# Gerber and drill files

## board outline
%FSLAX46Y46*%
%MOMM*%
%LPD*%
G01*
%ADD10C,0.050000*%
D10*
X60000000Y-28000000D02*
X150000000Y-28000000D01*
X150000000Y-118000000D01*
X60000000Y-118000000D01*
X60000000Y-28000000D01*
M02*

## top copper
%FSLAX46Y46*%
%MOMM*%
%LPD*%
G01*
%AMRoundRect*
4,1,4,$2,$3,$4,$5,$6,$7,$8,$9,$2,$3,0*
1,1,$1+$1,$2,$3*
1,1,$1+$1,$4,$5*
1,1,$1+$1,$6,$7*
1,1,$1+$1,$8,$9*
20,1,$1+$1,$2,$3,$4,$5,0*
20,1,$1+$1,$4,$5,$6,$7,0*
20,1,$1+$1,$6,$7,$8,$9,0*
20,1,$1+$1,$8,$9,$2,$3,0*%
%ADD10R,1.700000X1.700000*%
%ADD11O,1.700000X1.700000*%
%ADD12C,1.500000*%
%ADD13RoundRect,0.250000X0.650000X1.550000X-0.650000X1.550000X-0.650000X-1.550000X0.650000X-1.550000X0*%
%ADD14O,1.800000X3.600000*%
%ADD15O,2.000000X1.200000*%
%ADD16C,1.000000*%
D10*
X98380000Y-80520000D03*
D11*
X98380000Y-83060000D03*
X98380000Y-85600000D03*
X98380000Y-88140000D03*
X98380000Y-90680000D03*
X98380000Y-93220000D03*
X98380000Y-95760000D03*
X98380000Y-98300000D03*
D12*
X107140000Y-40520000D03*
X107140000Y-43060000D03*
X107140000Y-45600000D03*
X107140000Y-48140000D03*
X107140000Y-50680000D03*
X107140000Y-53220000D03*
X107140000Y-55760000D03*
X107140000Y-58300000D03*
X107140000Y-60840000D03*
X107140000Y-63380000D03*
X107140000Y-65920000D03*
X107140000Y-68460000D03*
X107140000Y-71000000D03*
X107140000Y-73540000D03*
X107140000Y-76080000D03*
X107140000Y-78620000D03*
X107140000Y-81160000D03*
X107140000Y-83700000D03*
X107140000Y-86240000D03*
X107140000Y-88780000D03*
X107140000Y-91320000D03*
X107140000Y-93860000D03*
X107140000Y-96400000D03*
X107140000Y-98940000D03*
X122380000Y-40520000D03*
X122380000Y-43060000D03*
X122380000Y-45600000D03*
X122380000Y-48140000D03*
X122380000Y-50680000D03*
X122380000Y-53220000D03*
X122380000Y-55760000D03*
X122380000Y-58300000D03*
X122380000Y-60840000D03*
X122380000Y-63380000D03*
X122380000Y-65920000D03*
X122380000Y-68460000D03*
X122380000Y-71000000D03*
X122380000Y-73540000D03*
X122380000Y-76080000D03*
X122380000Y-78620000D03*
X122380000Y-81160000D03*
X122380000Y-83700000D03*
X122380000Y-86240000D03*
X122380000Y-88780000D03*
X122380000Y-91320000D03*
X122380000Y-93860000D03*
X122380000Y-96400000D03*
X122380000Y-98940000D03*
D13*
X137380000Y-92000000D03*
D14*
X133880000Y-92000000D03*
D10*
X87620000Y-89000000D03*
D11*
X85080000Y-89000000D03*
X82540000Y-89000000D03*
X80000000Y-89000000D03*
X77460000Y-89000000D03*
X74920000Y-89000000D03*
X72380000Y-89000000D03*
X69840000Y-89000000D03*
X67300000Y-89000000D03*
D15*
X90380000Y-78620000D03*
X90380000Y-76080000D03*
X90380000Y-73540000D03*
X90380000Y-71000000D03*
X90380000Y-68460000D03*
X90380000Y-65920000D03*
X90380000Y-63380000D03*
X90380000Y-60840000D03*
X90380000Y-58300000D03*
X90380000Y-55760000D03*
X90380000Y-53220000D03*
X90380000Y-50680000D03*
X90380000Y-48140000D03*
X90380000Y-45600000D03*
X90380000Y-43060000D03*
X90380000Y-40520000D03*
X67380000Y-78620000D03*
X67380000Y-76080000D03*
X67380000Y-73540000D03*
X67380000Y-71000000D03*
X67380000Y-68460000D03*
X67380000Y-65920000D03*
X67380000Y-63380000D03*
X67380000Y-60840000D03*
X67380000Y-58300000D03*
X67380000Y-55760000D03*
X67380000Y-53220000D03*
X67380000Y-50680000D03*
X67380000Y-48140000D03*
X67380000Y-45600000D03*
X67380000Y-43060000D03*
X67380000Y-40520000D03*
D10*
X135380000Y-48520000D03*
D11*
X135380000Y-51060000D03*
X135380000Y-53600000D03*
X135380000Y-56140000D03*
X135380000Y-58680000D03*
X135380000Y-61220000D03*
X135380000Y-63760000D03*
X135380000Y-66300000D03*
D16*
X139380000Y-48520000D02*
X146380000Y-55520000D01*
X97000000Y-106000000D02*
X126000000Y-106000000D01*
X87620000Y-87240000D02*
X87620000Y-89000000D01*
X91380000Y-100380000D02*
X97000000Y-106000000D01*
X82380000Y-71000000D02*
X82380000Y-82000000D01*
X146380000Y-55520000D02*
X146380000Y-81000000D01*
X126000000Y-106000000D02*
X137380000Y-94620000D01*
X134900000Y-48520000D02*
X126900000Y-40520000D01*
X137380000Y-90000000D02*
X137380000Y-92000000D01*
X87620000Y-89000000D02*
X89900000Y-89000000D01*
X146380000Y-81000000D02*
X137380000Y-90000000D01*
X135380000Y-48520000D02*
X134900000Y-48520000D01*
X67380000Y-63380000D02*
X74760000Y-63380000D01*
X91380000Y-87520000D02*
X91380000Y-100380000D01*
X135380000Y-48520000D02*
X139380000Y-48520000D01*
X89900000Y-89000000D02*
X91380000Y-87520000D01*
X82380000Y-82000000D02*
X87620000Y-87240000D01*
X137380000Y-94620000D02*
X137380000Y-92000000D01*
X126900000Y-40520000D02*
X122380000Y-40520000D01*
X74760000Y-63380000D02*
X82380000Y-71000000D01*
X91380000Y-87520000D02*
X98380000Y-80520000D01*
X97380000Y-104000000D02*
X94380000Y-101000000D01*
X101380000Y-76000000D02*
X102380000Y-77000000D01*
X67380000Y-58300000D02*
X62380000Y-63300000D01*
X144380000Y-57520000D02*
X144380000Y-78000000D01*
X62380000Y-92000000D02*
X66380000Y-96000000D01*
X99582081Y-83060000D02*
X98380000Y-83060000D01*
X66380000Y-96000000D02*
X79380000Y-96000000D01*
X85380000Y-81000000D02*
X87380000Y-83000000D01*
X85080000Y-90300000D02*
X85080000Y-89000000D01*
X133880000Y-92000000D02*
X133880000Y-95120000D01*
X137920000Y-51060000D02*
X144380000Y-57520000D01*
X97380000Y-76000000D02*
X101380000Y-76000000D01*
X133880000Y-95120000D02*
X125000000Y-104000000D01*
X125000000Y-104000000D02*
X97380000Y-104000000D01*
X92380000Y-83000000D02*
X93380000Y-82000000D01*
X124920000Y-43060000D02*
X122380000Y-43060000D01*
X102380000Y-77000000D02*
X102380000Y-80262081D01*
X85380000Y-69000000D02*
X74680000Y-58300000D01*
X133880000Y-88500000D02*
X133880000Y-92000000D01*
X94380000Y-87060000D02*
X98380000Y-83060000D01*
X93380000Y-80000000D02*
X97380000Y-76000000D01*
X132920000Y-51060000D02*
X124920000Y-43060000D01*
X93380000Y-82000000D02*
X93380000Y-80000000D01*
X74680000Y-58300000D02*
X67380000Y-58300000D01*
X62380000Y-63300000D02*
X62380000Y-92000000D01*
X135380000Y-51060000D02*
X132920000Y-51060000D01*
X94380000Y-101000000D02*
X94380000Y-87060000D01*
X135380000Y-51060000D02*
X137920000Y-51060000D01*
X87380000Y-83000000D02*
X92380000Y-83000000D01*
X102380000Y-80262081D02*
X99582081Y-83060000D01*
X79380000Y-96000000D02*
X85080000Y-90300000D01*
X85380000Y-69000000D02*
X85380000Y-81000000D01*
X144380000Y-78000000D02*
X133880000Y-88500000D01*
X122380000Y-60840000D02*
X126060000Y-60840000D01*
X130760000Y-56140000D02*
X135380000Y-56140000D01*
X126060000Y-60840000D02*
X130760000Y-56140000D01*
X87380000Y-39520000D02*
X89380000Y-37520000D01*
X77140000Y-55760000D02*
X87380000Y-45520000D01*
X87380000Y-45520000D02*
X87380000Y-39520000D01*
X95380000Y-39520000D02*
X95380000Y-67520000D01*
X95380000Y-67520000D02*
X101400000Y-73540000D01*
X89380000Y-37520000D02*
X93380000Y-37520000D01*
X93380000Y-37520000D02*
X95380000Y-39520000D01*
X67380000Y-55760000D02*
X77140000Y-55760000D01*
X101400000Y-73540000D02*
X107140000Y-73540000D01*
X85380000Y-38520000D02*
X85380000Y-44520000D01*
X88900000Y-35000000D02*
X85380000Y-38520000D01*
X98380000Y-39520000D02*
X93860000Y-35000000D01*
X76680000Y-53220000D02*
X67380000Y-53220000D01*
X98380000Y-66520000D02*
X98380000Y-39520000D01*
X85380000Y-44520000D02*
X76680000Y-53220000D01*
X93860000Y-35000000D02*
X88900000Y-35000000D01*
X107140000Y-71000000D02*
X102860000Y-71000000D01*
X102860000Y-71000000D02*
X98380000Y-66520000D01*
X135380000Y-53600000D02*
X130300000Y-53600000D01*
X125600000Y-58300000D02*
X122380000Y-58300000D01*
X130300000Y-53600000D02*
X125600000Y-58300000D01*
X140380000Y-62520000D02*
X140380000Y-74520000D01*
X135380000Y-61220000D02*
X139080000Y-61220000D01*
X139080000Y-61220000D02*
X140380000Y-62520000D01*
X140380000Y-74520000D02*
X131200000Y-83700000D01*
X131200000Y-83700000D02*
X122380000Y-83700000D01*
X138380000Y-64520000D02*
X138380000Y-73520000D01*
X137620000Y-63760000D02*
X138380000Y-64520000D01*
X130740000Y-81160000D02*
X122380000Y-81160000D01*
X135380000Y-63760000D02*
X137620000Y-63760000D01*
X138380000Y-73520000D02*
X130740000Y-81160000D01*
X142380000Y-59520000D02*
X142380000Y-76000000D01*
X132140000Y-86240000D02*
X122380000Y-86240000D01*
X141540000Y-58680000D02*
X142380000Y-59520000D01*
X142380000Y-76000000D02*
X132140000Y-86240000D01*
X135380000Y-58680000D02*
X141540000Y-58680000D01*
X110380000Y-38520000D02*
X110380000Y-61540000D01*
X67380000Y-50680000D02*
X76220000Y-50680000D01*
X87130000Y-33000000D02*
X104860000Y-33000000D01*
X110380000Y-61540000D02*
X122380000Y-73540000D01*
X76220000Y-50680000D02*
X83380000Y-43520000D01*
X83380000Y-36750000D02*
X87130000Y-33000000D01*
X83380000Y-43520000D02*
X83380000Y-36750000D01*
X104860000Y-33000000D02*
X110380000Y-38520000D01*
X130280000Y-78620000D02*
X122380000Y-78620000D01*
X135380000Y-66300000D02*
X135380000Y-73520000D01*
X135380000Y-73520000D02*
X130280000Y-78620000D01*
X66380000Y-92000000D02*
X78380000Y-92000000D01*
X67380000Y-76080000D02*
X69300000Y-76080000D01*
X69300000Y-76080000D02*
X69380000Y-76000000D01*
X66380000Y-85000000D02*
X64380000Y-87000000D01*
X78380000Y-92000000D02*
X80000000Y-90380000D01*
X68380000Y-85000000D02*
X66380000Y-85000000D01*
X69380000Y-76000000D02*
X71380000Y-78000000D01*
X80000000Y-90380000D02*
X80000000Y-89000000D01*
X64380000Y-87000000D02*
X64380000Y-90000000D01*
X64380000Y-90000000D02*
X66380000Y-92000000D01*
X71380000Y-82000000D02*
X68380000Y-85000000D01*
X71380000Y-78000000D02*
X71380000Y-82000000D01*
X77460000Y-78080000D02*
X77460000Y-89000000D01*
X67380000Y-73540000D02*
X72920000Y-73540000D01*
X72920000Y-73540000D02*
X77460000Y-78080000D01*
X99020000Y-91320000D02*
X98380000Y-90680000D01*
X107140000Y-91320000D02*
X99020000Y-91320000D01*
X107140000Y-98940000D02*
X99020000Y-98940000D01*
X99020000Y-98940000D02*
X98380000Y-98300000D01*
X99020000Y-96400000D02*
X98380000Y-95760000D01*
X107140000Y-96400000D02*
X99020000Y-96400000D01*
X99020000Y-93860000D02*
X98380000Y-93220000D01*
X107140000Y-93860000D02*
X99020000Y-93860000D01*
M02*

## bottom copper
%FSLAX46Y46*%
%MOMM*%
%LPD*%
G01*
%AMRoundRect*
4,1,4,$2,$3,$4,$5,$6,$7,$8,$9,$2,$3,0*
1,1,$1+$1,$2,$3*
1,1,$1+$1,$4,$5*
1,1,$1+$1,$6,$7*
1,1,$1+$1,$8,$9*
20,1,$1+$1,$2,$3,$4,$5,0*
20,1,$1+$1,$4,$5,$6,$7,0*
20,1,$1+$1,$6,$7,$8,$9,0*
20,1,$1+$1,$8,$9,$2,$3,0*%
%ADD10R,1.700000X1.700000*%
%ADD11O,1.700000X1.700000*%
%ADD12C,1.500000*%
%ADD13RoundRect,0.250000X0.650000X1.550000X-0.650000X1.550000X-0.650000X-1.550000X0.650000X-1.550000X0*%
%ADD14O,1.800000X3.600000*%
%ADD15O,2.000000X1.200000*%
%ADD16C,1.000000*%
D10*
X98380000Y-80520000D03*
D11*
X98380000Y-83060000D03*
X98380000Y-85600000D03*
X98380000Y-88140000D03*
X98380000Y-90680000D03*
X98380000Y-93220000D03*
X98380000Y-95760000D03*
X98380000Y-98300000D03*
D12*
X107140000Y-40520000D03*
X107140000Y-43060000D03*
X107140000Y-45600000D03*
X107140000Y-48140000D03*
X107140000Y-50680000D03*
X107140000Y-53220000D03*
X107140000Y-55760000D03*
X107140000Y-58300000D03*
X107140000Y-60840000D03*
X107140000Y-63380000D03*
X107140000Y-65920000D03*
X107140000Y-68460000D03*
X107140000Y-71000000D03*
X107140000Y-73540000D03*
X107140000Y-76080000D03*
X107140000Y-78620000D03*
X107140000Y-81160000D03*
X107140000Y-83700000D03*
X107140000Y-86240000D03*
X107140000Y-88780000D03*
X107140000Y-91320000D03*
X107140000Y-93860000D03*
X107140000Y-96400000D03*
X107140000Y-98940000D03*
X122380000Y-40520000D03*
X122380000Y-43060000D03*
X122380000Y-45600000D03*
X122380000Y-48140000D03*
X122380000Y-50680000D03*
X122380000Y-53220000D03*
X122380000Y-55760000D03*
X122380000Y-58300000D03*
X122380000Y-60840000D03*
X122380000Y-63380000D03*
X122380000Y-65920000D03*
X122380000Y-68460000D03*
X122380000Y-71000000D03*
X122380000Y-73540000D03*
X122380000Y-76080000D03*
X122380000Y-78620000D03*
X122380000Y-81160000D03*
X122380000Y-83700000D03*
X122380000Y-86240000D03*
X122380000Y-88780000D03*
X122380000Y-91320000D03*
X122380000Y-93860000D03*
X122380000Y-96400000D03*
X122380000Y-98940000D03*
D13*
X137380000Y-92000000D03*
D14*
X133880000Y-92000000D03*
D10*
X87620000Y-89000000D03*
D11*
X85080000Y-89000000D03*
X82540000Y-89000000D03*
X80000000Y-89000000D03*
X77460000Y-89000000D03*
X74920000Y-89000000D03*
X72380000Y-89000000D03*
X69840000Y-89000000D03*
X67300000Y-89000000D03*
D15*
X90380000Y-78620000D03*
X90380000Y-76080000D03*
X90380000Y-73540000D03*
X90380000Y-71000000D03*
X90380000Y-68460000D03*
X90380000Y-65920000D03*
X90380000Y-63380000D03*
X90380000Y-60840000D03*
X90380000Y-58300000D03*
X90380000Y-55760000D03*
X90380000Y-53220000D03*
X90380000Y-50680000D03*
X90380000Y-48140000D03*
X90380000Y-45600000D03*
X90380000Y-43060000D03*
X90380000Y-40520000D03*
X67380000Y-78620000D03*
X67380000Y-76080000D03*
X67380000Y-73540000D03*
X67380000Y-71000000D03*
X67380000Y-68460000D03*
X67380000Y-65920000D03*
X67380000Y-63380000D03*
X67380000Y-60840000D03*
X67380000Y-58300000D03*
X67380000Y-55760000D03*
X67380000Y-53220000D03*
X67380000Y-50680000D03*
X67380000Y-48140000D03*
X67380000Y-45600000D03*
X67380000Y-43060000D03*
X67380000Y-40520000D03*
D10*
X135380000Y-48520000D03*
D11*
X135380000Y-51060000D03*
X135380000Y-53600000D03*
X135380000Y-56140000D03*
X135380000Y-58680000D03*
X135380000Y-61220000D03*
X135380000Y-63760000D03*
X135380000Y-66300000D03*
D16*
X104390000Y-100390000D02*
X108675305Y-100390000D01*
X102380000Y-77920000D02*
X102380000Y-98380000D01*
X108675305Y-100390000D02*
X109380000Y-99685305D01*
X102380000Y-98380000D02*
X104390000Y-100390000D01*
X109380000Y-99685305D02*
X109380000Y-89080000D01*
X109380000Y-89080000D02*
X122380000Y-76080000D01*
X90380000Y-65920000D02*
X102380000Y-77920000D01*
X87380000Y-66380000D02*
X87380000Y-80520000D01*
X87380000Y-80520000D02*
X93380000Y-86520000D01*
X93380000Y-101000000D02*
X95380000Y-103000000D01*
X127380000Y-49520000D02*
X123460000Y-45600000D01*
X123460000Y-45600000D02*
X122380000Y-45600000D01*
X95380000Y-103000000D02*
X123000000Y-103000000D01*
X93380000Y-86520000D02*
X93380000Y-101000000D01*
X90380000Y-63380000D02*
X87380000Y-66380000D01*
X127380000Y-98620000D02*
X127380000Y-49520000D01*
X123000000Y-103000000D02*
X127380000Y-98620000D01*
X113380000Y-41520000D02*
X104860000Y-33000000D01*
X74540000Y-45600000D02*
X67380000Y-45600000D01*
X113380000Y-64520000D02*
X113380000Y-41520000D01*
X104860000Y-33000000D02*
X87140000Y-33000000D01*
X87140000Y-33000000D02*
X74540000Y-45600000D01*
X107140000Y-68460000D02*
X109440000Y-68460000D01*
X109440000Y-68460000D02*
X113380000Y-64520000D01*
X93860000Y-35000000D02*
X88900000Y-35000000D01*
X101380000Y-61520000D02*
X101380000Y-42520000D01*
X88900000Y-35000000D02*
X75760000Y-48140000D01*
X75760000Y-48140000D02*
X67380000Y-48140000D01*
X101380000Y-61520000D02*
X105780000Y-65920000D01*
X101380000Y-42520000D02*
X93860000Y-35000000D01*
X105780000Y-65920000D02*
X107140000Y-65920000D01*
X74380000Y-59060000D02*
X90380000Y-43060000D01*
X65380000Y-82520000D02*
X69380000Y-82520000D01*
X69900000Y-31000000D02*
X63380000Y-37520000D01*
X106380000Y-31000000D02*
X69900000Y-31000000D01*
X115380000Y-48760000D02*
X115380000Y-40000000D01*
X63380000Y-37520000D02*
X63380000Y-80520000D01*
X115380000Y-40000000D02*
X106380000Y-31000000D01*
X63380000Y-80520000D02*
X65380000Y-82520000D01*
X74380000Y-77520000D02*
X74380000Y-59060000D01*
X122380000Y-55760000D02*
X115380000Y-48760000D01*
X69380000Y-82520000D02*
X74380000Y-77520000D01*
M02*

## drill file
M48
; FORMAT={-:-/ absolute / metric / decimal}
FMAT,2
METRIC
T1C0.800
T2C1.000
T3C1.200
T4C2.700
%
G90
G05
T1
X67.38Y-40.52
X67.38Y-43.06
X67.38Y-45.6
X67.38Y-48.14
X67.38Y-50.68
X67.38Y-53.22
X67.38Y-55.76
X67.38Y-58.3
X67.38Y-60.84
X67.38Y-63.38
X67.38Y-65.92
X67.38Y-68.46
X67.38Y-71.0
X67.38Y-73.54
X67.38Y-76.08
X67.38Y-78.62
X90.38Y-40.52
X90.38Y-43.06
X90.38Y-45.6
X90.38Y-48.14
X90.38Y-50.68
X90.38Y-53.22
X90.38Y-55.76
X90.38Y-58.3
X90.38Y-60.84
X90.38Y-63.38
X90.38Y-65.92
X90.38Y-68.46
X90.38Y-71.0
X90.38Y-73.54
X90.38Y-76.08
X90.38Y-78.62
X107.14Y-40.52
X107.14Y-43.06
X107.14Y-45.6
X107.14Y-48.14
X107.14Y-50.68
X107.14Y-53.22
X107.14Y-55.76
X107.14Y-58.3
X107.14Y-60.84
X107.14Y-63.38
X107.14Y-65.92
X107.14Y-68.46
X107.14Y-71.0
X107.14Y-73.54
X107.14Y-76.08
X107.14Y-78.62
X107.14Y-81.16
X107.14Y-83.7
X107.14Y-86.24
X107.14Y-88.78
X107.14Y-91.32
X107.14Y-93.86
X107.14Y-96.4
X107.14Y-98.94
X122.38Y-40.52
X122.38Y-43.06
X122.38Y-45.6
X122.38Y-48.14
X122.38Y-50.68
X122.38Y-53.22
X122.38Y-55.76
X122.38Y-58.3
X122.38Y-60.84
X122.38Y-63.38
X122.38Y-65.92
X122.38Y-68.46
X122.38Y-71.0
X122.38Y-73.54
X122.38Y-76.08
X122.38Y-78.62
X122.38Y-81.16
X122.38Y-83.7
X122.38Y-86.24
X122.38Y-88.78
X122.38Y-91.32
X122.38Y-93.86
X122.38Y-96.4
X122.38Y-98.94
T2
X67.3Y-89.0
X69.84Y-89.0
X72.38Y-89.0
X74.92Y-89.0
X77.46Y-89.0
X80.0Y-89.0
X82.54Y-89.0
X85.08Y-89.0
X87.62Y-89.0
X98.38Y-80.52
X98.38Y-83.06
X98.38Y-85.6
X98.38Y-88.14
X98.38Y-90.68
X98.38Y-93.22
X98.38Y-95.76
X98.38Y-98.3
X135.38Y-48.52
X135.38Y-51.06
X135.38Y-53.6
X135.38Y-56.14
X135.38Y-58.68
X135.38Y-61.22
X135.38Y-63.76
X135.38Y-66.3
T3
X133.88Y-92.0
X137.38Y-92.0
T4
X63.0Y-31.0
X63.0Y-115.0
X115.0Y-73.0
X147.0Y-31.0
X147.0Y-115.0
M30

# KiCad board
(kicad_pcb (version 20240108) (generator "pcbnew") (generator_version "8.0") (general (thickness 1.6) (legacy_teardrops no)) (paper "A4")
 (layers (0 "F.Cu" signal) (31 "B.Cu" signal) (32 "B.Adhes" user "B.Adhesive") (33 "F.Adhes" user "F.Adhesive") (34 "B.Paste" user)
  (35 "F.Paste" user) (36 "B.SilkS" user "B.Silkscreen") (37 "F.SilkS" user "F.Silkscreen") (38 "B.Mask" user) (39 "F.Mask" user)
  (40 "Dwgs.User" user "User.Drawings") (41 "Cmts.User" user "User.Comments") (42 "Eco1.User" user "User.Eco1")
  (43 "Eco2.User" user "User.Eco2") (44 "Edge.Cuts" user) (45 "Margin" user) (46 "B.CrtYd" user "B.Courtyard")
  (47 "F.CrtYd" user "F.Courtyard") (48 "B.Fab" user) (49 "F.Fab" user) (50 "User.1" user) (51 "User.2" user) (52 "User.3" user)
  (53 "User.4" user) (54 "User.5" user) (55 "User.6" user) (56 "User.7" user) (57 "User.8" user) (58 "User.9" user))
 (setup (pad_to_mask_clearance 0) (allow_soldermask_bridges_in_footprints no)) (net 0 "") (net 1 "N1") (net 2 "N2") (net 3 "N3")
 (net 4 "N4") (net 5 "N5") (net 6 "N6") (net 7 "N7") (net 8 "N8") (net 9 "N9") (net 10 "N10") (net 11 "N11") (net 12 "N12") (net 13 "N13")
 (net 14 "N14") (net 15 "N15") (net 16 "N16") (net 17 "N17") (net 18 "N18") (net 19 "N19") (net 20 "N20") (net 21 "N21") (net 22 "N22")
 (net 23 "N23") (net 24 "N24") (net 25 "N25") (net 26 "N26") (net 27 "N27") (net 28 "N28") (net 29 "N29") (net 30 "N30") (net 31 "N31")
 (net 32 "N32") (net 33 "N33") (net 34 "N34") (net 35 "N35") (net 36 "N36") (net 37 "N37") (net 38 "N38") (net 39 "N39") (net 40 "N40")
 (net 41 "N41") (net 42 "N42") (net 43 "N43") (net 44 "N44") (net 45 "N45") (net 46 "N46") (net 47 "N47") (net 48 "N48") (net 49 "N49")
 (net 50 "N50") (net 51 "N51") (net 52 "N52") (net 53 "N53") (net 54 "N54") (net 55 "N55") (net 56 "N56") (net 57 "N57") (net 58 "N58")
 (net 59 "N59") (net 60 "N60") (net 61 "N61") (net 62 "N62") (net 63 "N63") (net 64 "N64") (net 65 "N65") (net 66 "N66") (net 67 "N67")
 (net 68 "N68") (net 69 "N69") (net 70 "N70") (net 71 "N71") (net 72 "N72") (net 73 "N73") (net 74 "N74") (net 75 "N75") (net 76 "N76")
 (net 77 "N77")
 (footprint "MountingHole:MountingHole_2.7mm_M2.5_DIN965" (layer "F.Cu") (at 63 115)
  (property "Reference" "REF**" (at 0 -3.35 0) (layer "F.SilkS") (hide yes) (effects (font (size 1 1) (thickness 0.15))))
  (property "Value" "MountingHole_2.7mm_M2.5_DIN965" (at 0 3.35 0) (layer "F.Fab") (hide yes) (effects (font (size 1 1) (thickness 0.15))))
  (pad "" np_thru_hole circle (at 0 0) (size 2.7 2.7) (drill 2.7) (layers "*.Cu" "*.Mask")))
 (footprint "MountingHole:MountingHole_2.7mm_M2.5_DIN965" (layer "F.Cu") (at 115 73)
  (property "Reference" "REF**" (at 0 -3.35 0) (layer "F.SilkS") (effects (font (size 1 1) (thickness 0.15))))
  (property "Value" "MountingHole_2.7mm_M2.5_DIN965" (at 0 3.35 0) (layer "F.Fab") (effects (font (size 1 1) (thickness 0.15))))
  (pad "" np_thru_hole circle (at 0 0) (size 2.7 2.7) (drill 2.7) (layers "F&B.Cu" "*.Mask")))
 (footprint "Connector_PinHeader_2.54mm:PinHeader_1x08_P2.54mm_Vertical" (layer "F.Cu") (at 98.38 80.52)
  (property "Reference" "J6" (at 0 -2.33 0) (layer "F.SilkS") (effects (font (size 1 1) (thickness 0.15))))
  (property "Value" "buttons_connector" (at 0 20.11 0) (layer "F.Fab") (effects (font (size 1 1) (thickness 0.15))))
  (pad "1" thru_hole rect (at 0 0) (size 1.7 1.7) (drill 1) (layers "*.Cu" "*.Mask") (remove_unused_layers no) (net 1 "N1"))
  (pad "2" thru_hole oval (at 0 2.54) (size 1.7 1.7) (drill 1) (layers "*.Cu" "*.Mask") (remove_unused_layers no) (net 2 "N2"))
  (pad "3" thru_hole oval (at 0 5.08) (size 1.7 1.7) (drill 1) (layers "*.Cu" "*.Mask") (remove_unused_layers no) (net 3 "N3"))
  (pad "4" thru_hole oval (at 0 7.62) (size 1.7 1.7) (drill 1) (layers "*.Cu" "*.Mask") (remove_unused_layers no) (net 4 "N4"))
  (pad "5" thru_hole oval (at 0 10.16) (size 1.7 1.7) (drill 1) (layers "*.Cu" "*.Mask") (remove_unused_layers no) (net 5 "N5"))
  (pad "6" thru_hole oval (at 0 12.7) (size 1.7 1.7) (drill 1) (layers "*.Cu" "*.Mask") (remove_unused_layers no) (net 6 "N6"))
  (pad "7" thru_hole oval (at 0 15.24) (size 1.7 1.7) (drill 1) (layers "*.Cu" "*.Mask") (remove_unused_layers no) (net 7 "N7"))
  (pad "8" thru_hole oval (at 0 17.78) (size 1.7 1.7) (drill 1) (layers "*.Cu" "*.Mask") (remove_unused_layers no) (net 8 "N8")))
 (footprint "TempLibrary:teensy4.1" (layer "F.Cu") (at 114.76 69.73 -90)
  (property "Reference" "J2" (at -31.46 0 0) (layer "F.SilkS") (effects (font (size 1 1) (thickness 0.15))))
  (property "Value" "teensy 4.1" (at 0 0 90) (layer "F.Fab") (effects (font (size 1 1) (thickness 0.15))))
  (pad "1" thru_hole circle (at -29.21 7.62 270) (size 1.5 1.5) (drill 0.8) (layers "*.Cu" "*.Mask") (remove_unused_layers no) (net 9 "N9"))
  (pad "2" thru_hole circle (at -26.67 7.62 270) (size 1.5 1.5) (drill 0.8) (layers "*.Cu" "*.Mask") (remove_unused_layers no)
   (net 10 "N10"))
  (pad "3" thru_hole circle (at -24.13 7.62 270) (size 1.5 1.5) (drill 0.8) (layers "*.Cu" "*.Mask") (remove_unused_layers no)
   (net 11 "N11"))
  (pad "4" thru_hole circle (at -21.59 7.62 270) (size 1.5 1.5) (drill 0.8) (layers "*.Cu" "*.Mask") (remove_unused_layers no)
   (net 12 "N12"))
  (pad "5" thru_hole circle (at -19.05 7.62 270) (size 1.5 1.5) (drill 0.8) (layers "*.Cu" "*.Mask") (remove_unused_layers no)
   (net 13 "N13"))
  (pad "6" thru_hole circle (at -16.51 7.62 270) (size 1.5 1.5) (drill 0.8) (layers "*.Cu" "*.Mask") (remove_unused_layers no)
   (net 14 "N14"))
  (pad "7" thru_hole circle (at -13.97 7.62 270) (size 1.5 1.5) (drill 0.8) (layers "*.Cu" "*.Mask") (remove_unused_layers no)
   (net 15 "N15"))
  (pad "8" thru_hole circle (at -11.43 7.62 270) (size 1.5 1.5) (drill 0.8) (layers "*.Cu" "*.Mask") (remove_unused_layers no)
   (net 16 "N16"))
  (pad "9" thru_hole circle (at -8.89 7.62 270) (size 1.5 1.5) (drill 0.8) (layers "*.Cu" "*.Mask") (remove_unused_layers no) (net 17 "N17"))
  (pad "10" thru_hole circle (at -6.35 7.62 270) (size 1.5 1.5) (drill 0.8) (layers "*.Cu" "*.Mask") (remove_unused_layers no)
   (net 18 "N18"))
  (pad "11" thru_hole circle (at -3.81 7.62 270) (size 1.5 1.5) (drill 0.8) (layers "*.Cu" "*.Mask") (remove_unused_layers no)
   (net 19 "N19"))
  (pad "12" thru_hole circle (at -1.27 7.62 270) (size 1.5 1.5) (drill 0.8) (layers "*.Cu" "*.Mask") (remove_unused_layers no)
   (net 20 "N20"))
  (pad "13" thru_hole circle (at 1.27 7.62 270) (size 1.5 1.5) (drill 0.8) (layers "*.Cu" "*.Mask") (remove_unused_layers no) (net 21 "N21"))
  (pad "14" thru_hole circle (at 3.81 7.62 270) (size 1.5 1.5) (drill 0.8) (layers "*.Cu" "*.Mask") (remove_unused_layers no) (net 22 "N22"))
  (pad "15" thru_hole circle (at 6.35 7.62 270) (size 1.5 1.5) (drill 0.8) (layers "*.Cu" "*.Mask") (remove_unused_layers no) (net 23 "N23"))
  (pad "16" thru_hole circle (at 8.89 7.62 270) (size 1.5 1.5) (drill 0.8) (layers "*.Cu" "*.Mask") (remove_unused_layers no) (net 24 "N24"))
  (pad "17" thru_hole circle (at 11.43 7.62 270) (size 1.5 1.5) (drill 0.8) (layers "*.Cu" "*.Mask") (remove_unused_layers no)
   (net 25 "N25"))
  (pad "18" thru_hole circle (at 13.97 7.62 270) (size 1.5 1.5) (drill 0.8) (layers "*.Cu" "*.Mask") (remove_unused_layers no)
   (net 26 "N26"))
  (pad "19" thru_hole circle (at 16.51 7.62 270) (size 1.5 1.5) (drill 0.8) (layers "*.Cu" "*.Mask") (remove_unused_layers no)
   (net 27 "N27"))
  (pad "20" thru_hole circle (at 19.05 7.62 270) (size 1.5 1.5) (drill 0.8) (layers "*.Cu" "*.Mask") (remove_unused_layers no)
   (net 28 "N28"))
  (pad "21" thru_hole circle (at 21.59 7.62 270) (size 1.5 1.5) (drill 0.8) (layers "*.Cu" "*.Mask") (remove_unused_layers no) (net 5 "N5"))
  (pad "22" thru_hole circle (at 24.13 7.62 270) (size 1.5 1.5) (drill 0.8) (layers "*.Cu" "*.Mask") (remove_unused_layers no) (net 6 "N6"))
  (pad "23" thru_hole circle (at 26.67 7.62 270) (size 1.5 1.5) (drill 0.8) (layers "*.Cu" "*.Mask") (remove_unused_layers no) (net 7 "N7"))
  (pad "24" thru_hole circle (at 29.21 7.62 270) (size 1.5 1.5) (drill 0.8) (layers "*.Cu" "*.Mask") (remove_unused_layers no) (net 8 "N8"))
  (pad "25" thru_hole circle (at -29.21 -7.62 270) (size 1.5 1.5) (drill 0.8) (layers "*.Cu" "*.Mask") (remove_unused_layers no)
   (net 1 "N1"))
  (pad "26" thru_hole circle (at -26.67 -7.62 270) (size 1.5 1.5) (drill 0.8) (layers "*.Cu" "*.Mask") (remove_unused_layers no)
   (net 2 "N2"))
  (pad "27" thru_hole circle (at -24.13 -7.62 270) (size 1.5 1.5) (drill 0.8) (layers "*.Cu" "*.Mask") (remove_unused_layers no)
   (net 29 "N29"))
  (pad "28" thru_hole circle (at -21.59 -7.62 270) (size 1.5 1.5) (drill 0.8) (layers "*.Cu" "*.Mask") (remove_unused_layers no)
   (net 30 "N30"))
  (pad "29" thru_hole circle (at -19.05 -7.62 270) (size 1.5 1.5) (drill 0.8) (layers "*.Cu" "*.Mask") (remove_unused_layers no)
   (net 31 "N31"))
  (pad "30" thru_hole circle (at -16.51 -7.62 270) (size 1.5 1.5) (drill 0.8) (layers "*.Cu" "*.Mask") (remove_unused_layers no)
   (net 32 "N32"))
  (pad "31" thru_hole circle (at -13.97 -7.62 270) (size 1.5 1.5) (drill 0.8) (layers "*.Cu" "*.Mask") (remove_unused_layers no)
   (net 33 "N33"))
  (pad "32" thru_hole circle (at -11.43 -7.62 270) (size 1.5 1.5) (drill 0.8) (layers "*.Cu" "*.Mask") (remove_unused_layers no)
   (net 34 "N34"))
  (pad "33" thru_hole circle (at -8.89 -7.62 270) (size 1.5 1.5) (drill 0.8) (layers "*.Cu" "*.Mask") (remove_unused_layers no)
   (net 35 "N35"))
  (pad "34" thru_hole circle (at -6.35 -7.62 270) (size 1.5 1.5) (drill 0.8) (layers "*.Cu" "*.Mask") (remove_unused_layers no)
   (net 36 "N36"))
  (pad "35" thru_hole circle (at -3.81 -7.62 270) (size 1.5 1.5) (drill 0.8) (layers "*.Cu" "*.Mask") (remove_unused_layers no)
   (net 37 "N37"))
  (pad "36" thru_hole circle (at -1.27 -7.62 270) (size 1.5 1.5) (drill 0.8) (layers "*.Cu" "*.Mask") (remove_unused_layers no)
   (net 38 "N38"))
  (pad "37" thru_hole circle (at 1.27 -7.62 270) (size 1.5 1.5) (drill 0.8) (layers "*.Cu" "*.Mask") (remove_unused_layers no)
   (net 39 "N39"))
  (pad "38" thru_hole circle (at 3.81 -7.62 270) (size 1.5 1.5) (drill 0.8) (layers "*.Cu" "*.Mask") (remove_unused_layers no)
   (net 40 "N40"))
  (pad "39" thru_hole circle (at 6.35 -7.62 270) (size 1.5 1.5) (drill 0.8) (layers "*.Cu" "*.Mask") (remove_unused_layers no)
   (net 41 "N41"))
  (pad "40" thru_hole circle (at 8.89 -7.62 270) (size 1.5 1.5) (drill 0.8) (layers "*.Cu" "*.Mask") (remove_unused_layers no)
   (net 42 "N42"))
  (pad "41" thru_hole circle (at 11.43 -7.62 270) (size 1.5 1.5) (drill 0.8) (layers "*.Cu" "*.Mask") (remove_unused_layers no)
   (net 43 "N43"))
  (pad "42" thru_hole circle (at 13.97 -7.62 270) (size 1.5 1.5) (drill 0.8) (layers "*.Cu" "*.Mask") (remove_unused_layers no)
   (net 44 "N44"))
  (pad "43" thru_hole circle (at 16.51 -7.62 270) (size 1.5 1.5) (drill 0.8) (layers "*.Cu" "*.Mask") (remove_unused_layers no)
   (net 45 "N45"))
  (pad "44" thru_hole circle (at 19.05 -7.62 270) (size 1.5 1.5) (drill 0.8) (layers "*.Cu" "*.Mask") (remove_unused_layers no)
   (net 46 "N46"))
  (pad "45" thru_hole circle (at 21.59 -7.62 270) (size 1.5 1.5) (drill 0.8) (layers "*.Cu" "*.Mask") (remove_unused_layers no)
   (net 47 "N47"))
  (pad "46" thru_hole circle (at 24.13 -7.62 270) (size 1.5 1.5) (drill 0.8) (layers "*.Cu" "*.Mask") (remove_unused_layers no)
   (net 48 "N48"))
  (pad "47" thru_hole circle (at 26.67 -7.62 270) (size 1.5 1.5) (drill 0.8) (layers "*.Cu" "*.Mask") (remove_unused_layers no)
   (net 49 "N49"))
  (pad "48" thru_hole circle (at 29.21 -7.62 270) (size 1.5 1.5) (drill 0.8) (layers "*.Cu" "*.Mask") (remove_unused_layers no)
   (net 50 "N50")))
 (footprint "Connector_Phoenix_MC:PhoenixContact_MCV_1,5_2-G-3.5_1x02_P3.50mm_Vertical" (layer "F.Cu") (at 137.38 92 180)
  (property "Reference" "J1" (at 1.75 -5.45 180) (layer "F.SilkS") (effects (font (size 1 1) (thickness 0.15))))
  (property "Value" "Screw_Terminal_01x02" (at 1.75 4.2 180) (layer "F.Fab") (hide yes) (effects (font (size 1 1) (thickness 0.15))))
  (pad "1" thru_hole roundrect (at 0 0 180) (size 1.8 3.6) (drill 1.2) (layers "*.Cu" "*.Mask") (remove_unused_layers no)
   (roundrect_rratio 0.138889) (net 1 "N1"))
  (pad "2" thru_hole oval (at 3.5 0 180) (size 1.8 3.6) (drill 1.2) (layers "*.Cu" "*.Mask") (remove_unused_layers no) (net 2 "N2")))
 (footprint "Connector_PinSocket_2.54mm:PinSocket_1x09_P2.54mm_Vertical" (layer "F.Cu") (at 87.62 89 -90)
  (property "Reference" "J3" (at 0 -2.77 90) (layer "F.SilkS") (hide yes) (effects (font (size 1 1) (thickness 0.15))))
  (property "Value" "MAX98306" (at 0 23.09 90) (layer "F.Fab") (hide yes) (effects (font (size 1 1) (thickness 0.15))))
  (pad "1" thru_hole rect (at 0 0 270) (size 1.7 1.7) (drill 1) (layers "*.Cu" "*.Mask") (remove_unused_layers no) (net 1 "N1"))
  (pad "2" thru_hole oval (at 0 2.54 270) (size 1.7 1.7) (drill 1) (layers "*.Cu" "*.Mask") (remove_unused_layers no) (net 2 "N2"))
  (pad "3" thru_hole oval (at 0 5.08 270) (size 1.7 1.7) (drill 1) (layers "*.Cu" "*.Mask") (remove_unused_layers no) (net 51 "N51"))
  (pad "4" thru_hole oval (at 0 7.62 270) (size 1.7 1.7) (drill 1) (layers "*.Cu" "*.Mask") (remove_unused_layers no) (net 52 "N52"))
  (pad "5" thru_hole oval (at 0 10.16 270) (size 1.7 1.7) (drill 1) (layers "*.Cu" "*.Mask") (remove_unused_layers no) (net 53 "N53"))
  (pad "6" thru_hole oval (at 0 12.7 270) (size 1.7 1.7) (drill 1) (layers "*.Cu" "*.Mask") (remove_unused_layers no) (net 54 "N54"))
  (pad "7" thru_hole oval (at 0 15.24 270) (size 1.7 1.7) (drill 1) (layers "*.Cu" "*.Mask") (remove_unused_layers no) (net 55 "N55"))
  (pad "8" thru_hole oval (at 0 17.78 270) (size 1.7 1.7) (drill 1) (layers "*.Cu" "*.Mask") (remove_unused_layers no) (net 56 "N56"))
  (pad "9" thru_hole oval (at 0 20.32 270) (size 1.7 1.7) (drill 1) (layers "*.Cu" "*.Mask") (remove_unused_layers no) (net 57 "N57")))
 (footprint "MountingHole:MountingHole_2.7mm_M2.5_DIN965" (layer "F.Cu") (at 147 115)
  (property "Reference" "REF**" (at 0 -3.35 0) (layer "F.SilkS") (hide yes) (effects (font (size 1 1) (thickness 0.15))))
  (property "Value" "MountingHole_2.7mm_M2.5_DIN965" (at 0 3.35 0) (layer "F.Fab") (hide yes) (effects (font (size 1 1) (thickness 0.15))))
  (pad "" np_thru_hole circle (at 0 0) (size 2.7 2.7) (drill 2.7) (layers "*.Cu" "*.Mask")))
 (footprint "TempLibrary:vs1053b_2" (layer "F.Cu") (at 78.88 59.57 90)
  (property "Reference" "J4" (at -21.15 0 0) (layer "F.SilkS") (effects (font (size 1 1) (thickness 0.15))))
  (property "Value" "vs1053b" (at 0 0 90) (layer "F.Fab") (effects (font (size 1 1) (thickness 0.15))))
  (pad "1" thru_hole oval (at -19.05 11.5 90) (size 1.2 2) (drill 0.8) (layers "*.Cu" "*.Mask") (remove_unused_layers no) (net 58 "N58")
   (thermal_bridge_angle 45))
  (pad "2" thru_hole oval (at -16.51 11.5 90) (size 1.2 2) (drill 0.8) (layers "*.Cu" "*.Mask") (remove_unused_layers no) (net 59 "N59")
   (thermal_bridge_angle 45))
  (pad "3" thru_hole oval (at -13.97 11.5 90) (size 1.2 2) (drill 0.8) (layers "*.Cu" "*.Mask") (remove_unused_layers no) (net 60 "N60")
   (thermal_bridge_angle 45))
  (pad "4" thru_hole oval (at -11.43 11.5 90) (size 1.2 2) (drill 0.8) (layers "*.Cu" "*.Mask") (remove_unused_layers no) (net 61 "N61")
   (thermal_bridge_angle 45))
  (pad "5" thru_hole oval (at -8.89 11.5 90) (size 1.2 2) (drill 0.8) (layers "*.Cu" "*.Mask") (remove_unused_layers no) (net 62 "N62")
   (thermal_bridge_angle 45))
  (pad "6" thru_hole oval (at -6.35 11.5 90) (size 1.2 2) (drill 0.8) (layers "*.Cu" "*.Mask") (remove_unused_layers no) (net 41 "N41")
   (thermal_bridge_angle 45))
  (pad "7" thru_hole oval (at -3.81 11.5 90) (size 1.2 2) (drill 0.8) (layers "*.Cu" "*.Mask") (remove_unused_layers no) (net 29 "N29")
   (thermal_bridge_angle 45))
  (pad "8" thru_hole oval (at -1.27 11.5 90) (size 1.2 2) (drill 0.8) (layers "*.Cu" "*.Mask") (remove_unused_layers no) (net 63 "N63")
   (thermal_bridge_angle 45))
  (pad "9" thru_hole oval (at 1.27 11.5 90) (size 1.2 2) (drill 0.8) (layers "*.Cu" "*.Mask") (remove_unused_layers no) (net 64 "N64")
   (thermal_bridge_angle 45))
  (pad "10" thru_hole oval (at 3.81 11.5 90) (size 1.2 2) (drill 0.8) (layers "*.Cu" "*.Mask") (remove_unused_layers no) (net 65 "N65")
   (thermal_bridge_angle 45))
  (pad "11" thru_hole oval (at 6.35 11.5 90) (size 1.2 2) (drill 0.8) (layers "*.Cu" "*.Mask") (remove_unused_layers no) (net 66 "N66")
   (thermal_bridge_angle 45))
  (pad "12" thru_hole oval (at 8.89 11.5 90) (size 1.2 2) (drill 0.8) (layers "*.Cu" "*.Mask") (remove_unused_layers no) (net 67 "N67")
   (thermal_bridge_angle 45))
  (pad "13" thru_hole oval (at 11.43 11.5 90) (size 1.2 2) (drill 0.8) (layers "*.Cu" "*.Mask") (remove_unused_layers no) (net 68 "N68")
   (thermal_bridge_angle 45))
  (pad "14" thru_hole oval (at 13.97 11.5 90) (size 1.2 2) (drill 0.8) (layers "*.Cu" "*.Mask") (remove_unused_layers no) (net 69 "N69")
   (thermal_bridge_angle 45))
  (pad "15" thru_hole oval (at 16.51 11.5 90) (size 1.2 2) (drill 0.8) (layers "*.Cu" "*.Mask") (remove_unused_layers no) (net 33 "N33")
   (thermal_bridge_angle 45))
  (pad "16" thru_hole oval (at 19.05 11.5 90) (size 1.2 2) (drill 0.8) (layers "*.Cu" "*.Mask") (remove_unused_layers no) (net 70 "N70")
   (thermal_bridge_angle 45))
  (pad "17" thru_hole oval (at -19.05 -11.5 90) (size 1.2 2) (drill 0.8) (layers "*.Cu" "*.Mask") (remove_unused_layers no) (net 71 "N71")
   (thermal_bridge_angle 45))
  (pad "18" thru_hole oval (at -16.51 -11.5 90) (size 1.2 2) (drill 0.8) (layers "*.Cu" "*.Mask") (remove_unused_layers no) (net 52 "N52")
   (thermal_bridge_angle 45))
  (pad "19" thru_hole oval (at -13.97 -11.5 90) (size 1.2 2) (drill 0.8) (layers "*.Cu" "*.Mask") (remove_unused_layers no) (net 53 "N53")
   (thermal_bridge_angle 45))
  (pad "20" thru_hole oval (at -11.43 -11.5 90) (size 1.2 2) (drill 0.8) (layers "*.Cu" "*.Mask") (remove_unused_layers no) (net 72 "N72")
   (thermal_bridge_angle 45))
  (pad "21" thru_hole oval (at -8.89 -11.5 90) (size 1.2 2) (drill 0.8) (layers "*.Cu" "*.Mask") (remove_unused_layers no) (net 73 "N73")
   (thermal_bridge_angle 45))
  (pad "22" thru_hole oval (at -6.35 -11.5 90) (size 1.2 2) (drill 0.8) (layers "*.Cu" "*.Mask") (remove_unused_layers no) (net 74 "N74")
   (thermal_bridge_angle 45))
  (pad "23" thru_hole oval (at -3.81 -11.5 90) (size 1.2 2) (drill 0.8) (layers "*.Cu" "*.Mask") (remove_unused_layers no) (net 1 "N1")
   (thermal_bridge_angle 45))
  (pad "24" thru_hole oval (at -1.27 -11.5 90) (size 1.2 2) (drill 0.8) (layers "*.Cu" "*.Mask") (remove_unused_layers no) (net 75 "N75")
   (thermal_bridge_angle 45))
  (pad "25" thru_hole oval (at 1.27 -11.5 90) (size 1.2 2) (drill 0.8) (layers "*.Cu" "*.Mask") (remove_unused_layers no) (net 2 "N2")
   (thermal_bridge_angle 45))
  (pad "26" thru_hole oval (at 3.81 -11.5 90) (size 1.2 2) (drill 0.8) (layers "*.Cu" "*.Mask") (remove_unused_layers no) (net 22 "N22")
   (thermal_bridge_angle 45))
  (pad "27" thru_hole oval (at 6.35 -11.5 90) (size 1.2 2) (drill 0.8) (layers "*.Cu" "*.Mask") (remove_unused_layers no) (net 21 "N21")
   (thermal_bridge_angle 45))
  (pad "28" thru_hole oval (at 8.89 -11.5 90) (size 1.2 2) (drill 0.8) (layers "*.Cu" "*.Mask") (remove_unused_layers no) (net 40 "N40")
   (thermal_bridge_angle 45))
  (pad "29" thru_hole oval (at 11.43 -11.5 90) (size 1.2 2) (drill 0.8) (layers "*.Cu" "*.Mask") (remove_unused_layers no) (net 19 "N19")
   (thermal_bridge_angle 45))
  (pad "30" thru_hole oval (at 13.97 -11.5 90) (size 1.2 2) (drill 0.8) (layers "*.Cu" "*.Mask") (remove_unused_layers no) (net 20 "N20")
   (thermal_bridge_angle 45))
  (pad "31" thru_hole oval (at 16.51 -11.5 90) (size 1.2 2) (drill 0.8) (layers "*.Cu" "*.Mask") (remove_unused_layers no) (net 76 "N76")
   (thermal_bridge_angle 45))
  (pad "32" thru_hole oval (at 19.05 -11.5 90) (size 1.2 2) (drill 0.8) (layers "*.Cu" "*.Mask") (remove_unused_layers no) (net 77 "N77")
   (thermal_bridge_angle 45)))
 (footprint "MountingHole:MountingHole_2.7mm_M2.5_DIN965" (layer "F.Cu") (at 63 31)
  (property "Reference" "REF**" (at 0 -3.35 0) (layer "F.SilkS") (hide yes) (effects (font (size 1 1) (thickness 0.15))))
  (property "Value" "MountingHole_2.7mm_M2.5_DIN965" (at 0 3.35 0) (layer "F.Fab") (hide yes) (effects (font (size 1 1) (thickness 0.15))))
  (pad "" np_thru_hole circle (at 0 0) (size 2.7 2.7) (drill 2.7) (layers "*.Cu" "*.Mask")))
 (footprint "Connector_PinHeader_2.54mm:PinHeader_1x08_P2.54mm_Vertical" (layer "F.Cu") (at 135.38 48.52)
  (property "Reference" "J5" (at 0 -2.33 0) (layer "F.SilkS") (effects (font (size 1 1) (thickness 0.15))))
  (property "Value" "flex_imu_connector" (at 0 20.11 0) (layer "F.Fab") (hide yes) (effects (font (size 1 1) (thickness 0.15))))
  (pad "1" thru_hole rect (at 0 0) (size 1.7 1.7) (drill 1) (layers "*.Cu" "*.Mask") (remove_unused_layers no) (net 1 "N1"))
  (pad "2" thru_hole oval (at 0 2.54) (size 1.7 1.7) (drill 1) (layers "*.Cu" "*.Mask") (remove_unused_layers no) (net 2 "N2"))
  (pad "3" thru_hole oval (at 0 5.08) (size 1.7 1.7) (drill 1) (layers "*.Cu" "*.Mask") (remove_unused_layers no) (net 34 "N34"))
  (pad "4" thru_hole oval (at 0 7.62) (size 1.7 1.7) (drill 1) (layers "*.Cu" "*.Mask") (remove_unused_layers no) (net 35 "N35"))
  (pad "5" thru_hole oval (at 0 10.16) (size 1.7 1.7) (drill 1) (layers "*.Cu" "*.Mask") (remove_unused_layers no) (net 45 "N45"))
  (pad "6" thru_hole oval (at 0 12.7) (size 1.7 1.7) (drill 1) (layers "*.Cu" "*.Mask") (remove_unused_layers no) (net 44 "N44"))
  (pad "7" thru_hole oval (at 0 15.24) (size 1.7 1.7) (drill 1) (layers "*.Cu" "*.Mask") (remove_unused_layers no) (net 43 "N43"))
  (pad "8" thru_hole oval (at 0 17.78) (size 1.7 1.7) (drill 1) (layers "*.Cu" "*.Mask") (remove_unused_layers no) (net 42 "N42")))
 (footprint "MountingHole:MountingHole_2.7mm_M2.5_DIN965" (layer "F.Cu") (at 147 31)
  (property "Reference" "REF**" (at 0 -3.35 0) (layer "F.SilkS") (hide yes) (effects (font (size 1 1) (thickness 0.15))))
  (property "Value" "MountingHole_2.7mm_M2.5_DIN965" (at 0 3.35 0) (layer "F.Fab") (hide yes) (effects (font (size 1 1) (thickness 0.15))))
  (pad "" np_thru_hole circle (at 0 0) (size 2.7 2.7) (drill 2.7) (layers "*.Cu" "*.Mask")))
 (gr_rect (start 60 28) (end 150 118) (stroke (width 0.05) (type default)) (fill none) (layer "Edge.Cuts"))
 (segment (start 139.38 48.52) (end 146.38 55.52) (width 1) (layer "F.Cu") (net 1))
 (segment (start 97 106) (end 126 106) (width 1) (layer "F.Cu") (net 1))
 (segment (start 87.62 87.24) (end 87.62 89) (width 1) (layer "F.Cu") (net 1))
 (segment (start 91.38 100.38) (end 97 106) (width 1) (layer "F.Cu") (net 1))
 (segment (start 82.38 71) (end 82.38 82) (width 1) (layer "F.Cu") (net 1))
 (segment (start 146.38 55.52) (end 146.38 81) (width 1) (layer "F.Cu") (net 1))
 (segment (start 126 106) (end 137.38 94.62) (width 1) (layer "F.Cu") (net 1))
 (segment (start 134.9 48.52) (end 126.9 40.52) (width 1) (layer "F.Cu") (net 1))
 (segment (start 137.38 90) (end 137.38 92) (width 1) (layer "F.Cu") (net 1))
 (segment (start 87.62 89) (end 89.9 89) (width 1) (layer "F.Cu") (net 1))
 (segment (start 146.38 81) (end 137.38 90) (width 1) (layer "F.Cu") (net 1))
 (segment (start 135.38 48.52) (end 134.9 48.52) (width 1) (layer "F.Cu") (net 1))
 (segment (start 67.38 63.38) (end 74.76 63.38) (width 1) (layer "F.Cu") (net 1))
 (segment (start 91.38 87.52) (end 91.38 100.38) (width 1) (layer "F.Cu") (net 1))
 (segment (start 135.38 48.52) (end 139.38 48.52) (width 1) (layer "F.Cu") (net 1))
 (segment (start 89.9 89) (end 91.38 87.52) (width 1) (layer "F.Cu") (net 1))
 (segment (start 82.38 82) (end 87.62 87.24) (width 1) (layer "F.Cu") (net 1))
 (segment (start 137.38 94.62) (end 137.38 92) (width 1) (layer "F.Cu") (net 1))
 (segment (start 126.9 40.52) (end 122.38 40.52) (width 1) (layer "F.Cu") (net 1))
 (segment (start 74.76 63.38) (end 82.38 71) (width 1) (layer "F.Cu") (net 1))
 (segment (start 91.38 87.52) (end 98.38 80.52) (width 1) (layer "F.Cu") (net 1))
 (segment (start 97.38 104) (end 94.38 101) (width 1) (layer "F.Cu") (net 2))
 (segment (start 101.38 76) (end 102.38 77) (width 1) (layer "F.Cu") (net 2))
 (segment (start 67.38 58.3) (end 62.38 63.3) (width 1) (layer "F.Cu") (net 2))
 (segment (start 144.38 57.52) (end 144.38 78) (width 1) (layer "F.Cu") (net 2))
 (segment (start 62.38 92) (end 66.38 96) (width 1) (layer "F.Cu") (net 2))
 (segment (start 99.582081 83.06) (end 98.38 83.06) (width 1) (layer "F.Cu") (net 2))
 (segment (start 66.38 96) (end 79.38 96) (width 1) (layer "F.Cu") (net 2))
 (segment (start 85.38 81) (end 87.38 83) (width 1) (layer "F.Cu") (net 2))
 (segment (start 85.08 90.3) (end 85.08 89) (width 1) (layer "F.Cu") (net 2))
 (segment (start 133.88 92) (end 133.88 95.12) (width 1) (layer "F.Cu") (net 2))
 (segment (start 137.92 51.06) (end 144.38 57.52) (width 1) (layer "F.Cu") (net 2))
 (segment (start 97.38 76) (end 101.38 76) (width 1) (layer "F.Cu") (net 2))
 (segment (start 133.88 95.12) (end 125 104) (width 1) (layer "F.Cu") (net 2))
 (segment (start 125 104) (end 97.38 104) (width 1) (layer "F.Cu") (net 2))
 (segment (start 92.38 83) (end 93.38 82) (width 1) (layer "F.Cu") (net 2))
 (segment (start 124.92 43.06) (end 122.38 43.06) (width 1) (layer "F.Cu") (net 2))
 (segment (start 102.38 77) (end 102.38 80.262081) (width 1) (layer "F.Cu") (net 2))
 (segment (start 85.38 69) (end 74.68 58.3) (width 1) (layer "F.Cu") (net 2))
 (segment (start 133.88 88.5) (end 133.88 92) (width 1) (layer "F.Cu") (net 2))
 (segment (start 94.38 87.06) (end 98.38 83.06) (width 1) (layer "F.Cu") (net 2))
 (segment (start 93.38 80) (end 97.38 76) (width 1) (layer "F.Cu") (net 2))
 (segment (start 132.92 51.06) (end 124.92 43.06) (width 1) (layer "F.Cu") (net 2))
 (segment (start 93.38 82) (end 93.38 80) (width 1) (layer "F.Cu") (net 2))
 (segment (start 74.68 58.3) (end 67.38 58.3) (width 1) (layer "F.Cu") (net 2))
 (segment (start 62.38 63.3) (end 62.38 92) (width 1) (layer "F.Cu") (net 2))
 (segment (start 135.38 51.06) (end 132.92 51.06) (width 1) (layer "F.Cu") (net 2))
 (segment (start 94.38 101) (end 94.38 87.06) (width 1) (layer "F.Cu") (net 2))
 (segment (start 135.38 51.06) (end 137.92 51.06) (width 1) (layer "F.Cu") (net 2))
 (segment (start 87.38 83) (end 92.38 83) (width 1) (layer "F.Cu") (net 2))
 (segment (start 102.38 80.262081) (end 99.582081 83.06) (width 1) (layer "F.Cu") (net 2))
 (segment (start 79.38 96) (end 85.08 90.3) (width 1) (layer "F.Cu") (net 2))
 (segment (start 85.38 69) (end 85.38 81) (width 1) (layer "F.Cu") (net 2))
 (segment (start 144.38 78) (end 133.88 88.5) (width 1) (layer "F.Cu") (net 2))
 (segment (start 122.38 60.84) (end 126.06 60.84) (width 1) (layer "F.Cu") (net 35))
 (segment (start 130.76 56.14) (end 135.38 56.14) (width 1) (layer "F.Cu") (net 35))
 (segment (start 126.06 60.84) (end 130.76 56.14) (width 1) (layer "F.Cu") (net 35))
 (segment (start 104.39 100.39) (end 108.675305 100.39) (width 1) (layer "B.Cu") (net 41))
 (segment (start 102.38 77.92) (end 102.38 98.38) (width 1) (layer "B.Cu") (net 41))
 (segment (start 108.675305 100.39) (end 109.38 99.685305) (width 1) (layer "B.Cu") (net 41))
 (segment (start 102.38 98.38) (end 104.39 100.39) (width 1) (layer "B.Cu") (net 41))
 (segment (start 109.38 99.685305) (end 109.38 89.08) (width 1) (layer "B.Cu") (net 41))
 (segment (start 109.38 89.08) (end 122.38 76.08) (width 1) (layer "B.Cu") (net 41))
 (segment (start 90.38 65.92) (end 102.38 77.92) (width 1) (layer "B.Cu") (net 41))
 (segment (start 87.38 66.38) (end 87.38 80.52) (width 1) (layer "B.Cu") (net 29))
 (segment (start 87.38 80.52) (end 93.38 86.52) (width 1) (layer "B.Cu") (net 29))
 (segment (start 93.38 101) (end 95.38 103) (width 1) (layer "B.Cu") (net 29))
 (segment (start 127.38 49.52) (end 123.46 45.6) (width 1) (layer "B.Cu") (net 29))
 (segment (start 123.46 45.6) (end 122.38 45.6) (width 1) (layer "B.Cu") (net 29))
 (segment (start 95.38 103) (end 123 103) (width 1) (layer "B.Cu") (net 29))
 (segment (start 93.38 86.52) (end 93.38 101) (width 1) (layer "B.Cu") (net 29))
 (segment (start 90.38 63.38) (end 87.38 66.38) (width 1) (layer "B.Cu") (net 29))
 (segment (start 127.38 98.62) (end 127.38 49.52) (width 1) (layer "B.Cu") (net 29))
 (segment (start 123 103) (end 127.38 98.62) (width 1) (layer "B.Cu") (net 29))
 (segment (start 87.38 39.52) (end 89.38 37.52) (width 1) (layer "F.Cu") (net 22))
 (segment (start 77.14 55.76) (end 87.38 45.52) (width 1) (layer "F.Cu") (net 22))
 (segment (start 87.38 45.52) (end 87.38 39.52) (width 1) (layer "F.Cu") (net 22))
 (segment (start 95.38 39.52) (end 95.38 67.52) (width 1) (layer "F.Cu") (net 22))
 (segment (start 95.38 67.52) (end 101.4 73.54) (width 1) (layer "F.Cu") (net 22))
 (segment (start 89.38 37.52) (end 93.38 37.52) (width 1) (layer "F.Cu") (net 22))
 (segment (start 93.38 37.52) (end 95.38 39.52) (width 1) (layer "F.Cu") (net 22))
 (segment (start 67.38 55.76) (end 77.14 55.76) (width 1) (layer "F.Cu") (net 22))
 (segment (start 101.4 73.54) (end 107.14 73.54) (width 1) (layer "F.Cu") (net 22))
 (segment (start 85.38 38.52) (end 85.38 44.52) (width 1) (layer "F.Cu") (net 21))
 (segment (start 88.9 35) (end 85.38 38.52) (width 1) (layer "F.Cu") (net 21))
 (segment (start 98.38 39.52) (end 93.86 35) (width 1) (layer "F.Cu") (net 21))
 (segment (start 76.68 53.22) (end 67.38 53.22) (width 1) (layer "F.Cu") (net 21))
 (segment (start 98.38 66.52) (end 98.38 39.52) (width 1) (layer "F.Cu") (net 21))
 (segment (start 85.38 44.52) (end 76.68 53.22) (width 1) (layer "F.Cu") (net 21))
 (segment (start 93.86 35) (end 88.9 35) (width 1) (layer "F.Cu") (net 21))
 (segment (start 107.14 71) (end 102.86 71) (width 1) (layer "F.Cu") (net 21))
 (segment (start 102.86 71) (end 98.38 66.52) (width 1) (layer "F.Cu") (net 21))
 (segment (start 135.38 53.6) (end 130.3 53.6) (width 1) (layer "F.Cu") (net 34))
 (segment (start 125.6 58.3) (end 122.38 58.3) (width 1) (layer "F.Cu") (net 34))
 (segment (start 130.3 53.6) (end 125.6 58.3) (width 1) (layer "F.Cu") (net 34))
 (segment (start 140.38 62.52) (end 140.38 74.52) (width 1) (layer "F.Cu") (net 44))
 (segment (start 135.38 61.22) (end 139.08 61.22) (width 1) (layer "F.Cu") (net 44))
 (segment (start 139.08 61.22) (end 140.38 62.52) (width 1) (layer "F.Cu") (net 44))
 (segment (start 140.38 74.52) (end 131.2 83.7) (width 1) (layer "F.Cu") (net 44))
 (segment (start 131.2 83.7) (end 122.38 83.7) (width 1) (layer "F.Cu") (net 44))
 (segment (start 138.38 64.52) (end 138.38 73.52) (width 1) (layer "F.Cu") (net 43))
 (segment (start 137.62 63.76) (end 138.38 64.52) (width 1) (layer "F.Cu") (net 43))
 (segment (start 130.74 81.16) (end 122.38 81.16) (width 1) (layer "F.Cu") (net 43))
 (segment (start 135.38 63.76) (end 137.62 63.76) (width 1) (layer "F.Cu") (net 43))
 (segment (start 138.38 73.52) (end 130.74 81.16) (width 1) (layer "F.Cu") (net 43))
 (segment (start 113.38 41.52) (end 104.86 33) (width 1) (layer "B.Cu") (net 20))
 (segment (start 74.54 45.6) (end 67.38 45.6) (width 1) (layer "B.Cu") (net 20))
 (segment (start 113.38 64.52) (end 113.38 41.52) (width 1) (layer "B.Cu") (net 20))
 (segment (start 104.86 33) (end 87.14 33) (width 1) (layer "B.Cu") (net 20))
 (segment (start 87.14 33) (end 74.54 45.6) (width 1) (layer "B.Cu") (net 20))
 (segment (start 107.14 68.46) (end 109.44 68.46) (width 1) (layer "B.Cu") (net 20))
 (segment (start 109.44 68.46) (end 113.38 64.52) (width 1) (layer "B.Cu") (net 20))
 (segment (start 142.38 59.52) (end 142.38 76) (width 1) (layer "F.Cu") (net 45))
 (segment (start 132.14 86.24) (end 122.38 86.24) (width 1) (layer "F.Cu") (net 45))
 (segment (start 141.54 58.68) (end 142.38 59.52) (width 1) (layer "F.Cu") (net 45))
 (segment (start 142.38 76) (end 132.14 86.24) (width 1) (layer "F.Cu") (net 45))
 (segment (start 135.38 58.68) (end 141.54 58.68) (width 1) (layer "F.Cu") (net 45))
 (segment (start 110.38 38.52) (end 110.38 61.54) (width 1) (layer "F.Cu") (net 40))
 (segment (start 67.38 50.68) (end 76.22 50.68) (width 1) (layer "F.Cu") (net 40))
 (segment (start 87.13 33) (end 104.86 33) (width 1) (layer "F.Cu") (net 40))
 (segment (start 110.38 61.54) (end 122.38 73.54) (width 1) (layer "F.Cu") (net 40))
 (segment (start 76.22 50.68) (end 83.38 43.52) (width 1) (layer "F.Cu") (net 40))
 (segment (start 83.38 36.75) (end 87.13 33) (width 1) (layer "F.Cu") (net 40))
 (segment (start 83.38 43.52) (end 83.38 36.75) (width 1) (layer "F.Cu") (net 40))
 (segment (start 104.86 33) (end 110.38 38.52) (width 1) (layer "F.Cu") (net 40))
 (segment (start 93.86 35) (end 88.9 35) (width 1) (layer "B.Cu") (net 19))
 (segment (start 101.38 61.52) (end 101.38 42.52) (width 1) (layer "B.Cu") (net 19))
 (segment (start 88.9 35) (end 75.76 48.14) (width 1) (layer "B.Cu") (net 19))
 (segment (start 75.76 48.14) (end 67.38 48.14) (width 1) (layer "B.Cu") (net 19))
 (segment (start 101.38 61.52) (end 105.78 65.92) (width 1) (layer "B.Cu") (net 19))
 (segment (start 101.38 42.52) (end 93.86 35) (width 1) (layer "B.Cu") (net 19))
 (segment (start 105.78 65.92) (end 107.14 65.92) (width 1) (layer "B.Cu") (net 19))
 (segment (start 130.28 78.62) (end 122.38 78.62) (width 1) (layer "F.Cu") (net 42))
 (segment (start 135.38 66.3) (end 135.38 73.52) (width 1) (layer "F.Cu") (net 42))
 (segment (start 135.38 73.52) (end 130.28 78.62) (width 1) (layer "F.Cu") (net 42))
 (segment (start 66.38 92) (end 78.38 92) (width 1) (layer "F.Cu") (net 52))
 (segment (start 67.38 76.08) (end 69.3 76.08) (width 1) (layer "F.Cu") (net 52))
 (segment (start 69.3 76.08) (end 69.38 76) (width 1) (layer "F.Cu") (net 52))
 (segment (start 66.38 85) (end 64.38 87) (width 1) (layer "F.Cu") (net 52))
 (segment (start 78.38 92) (end 80 90.38) (width 1) (layer "F.Cu") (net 52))
 (segment (start 68.38 85) (end 66.38 85) (width 1) (layer "F.Cu") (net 52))
 (segment (start 69.38 76) (end 71.38 78) (width 1) (layer "F.Cu") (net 52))
 (segment (start 80 90.38) (end 80 89) (width 1) (layer "F.Cu") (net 52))
 (segment (start 64.38 87) (end 64.38 90) (width 1) (layer "F.Cu") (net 52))
 (segment (start 64.38 90) (end 66.38 92) (width 1) (layer "F.Cu") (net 52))
 (segment (start 71.38 82) (end 68.38 85) (width 1) (layer "F.Cu") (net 52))
 (segment (start 71.38 78) (end 71.38 82) (width 1) (layer "F.Cu") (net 52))
 (segment (start 77.46 78.08) (end 77.46 89) (width 1) (layer "F.Cu") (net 53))
 (segment (start 67.38 73.54) (end 72.92 73.54) (width 1) (layer "F.Cu") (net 53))
 (segment (start 72.92 73.54) (end 77.46 78.08) (width 1) (layer "F.Cu") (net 53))
 (segment (start 99.02 91.32) (end 98.38 90.68) (width 1) (layer "F.Cu") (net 5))
 (segment (start 107.14 91.32) (end 99.02 91.32) (width 1) (layer "F.Cu") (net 5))
 (segment (start 107.14 98.94) (end 99.02 98.94) (width 1) (layer "F.Cu") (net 8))
 (segment (start 99.02 98.94) (end 98.38 98.3) (width 1) (layer "F.Cu") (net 8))
 (segment (start 99.02 96.4) (end 98.38 95.76) (width 1) (layer "F.Cu") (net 7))
 (segment (start 107.14 96.4) (end 99.02 96.4) (width 1) (layer "F.Cu") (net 7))
 (segment (start 99.02 93.86) (end 98.38 93.22) (width 1) (layer "F.Cu") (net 6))
 (segment (start 107.14 93.86) (end 99.02 93.86) (width 1) (layer "F.Cu") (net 6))
 (segment (start 74.38 59.06) (end 90.38 43.06) (width 1) (layer "B.Cu") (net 33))
 (segment (start 65.38 82.52) (end 69.38 82.52) (width 1) (layer "B.Cu") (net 33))
 (segment (start 69.9 31) (end 63.38 37.52) (width 1) (layer "B.Cu") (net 33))
 (segment (start 106.38 31) (end 69.9 31) (width 1) (layer "B.Cu") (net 33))
 (segment (start 115.38 48.76) (end 115.38 40) (width 1) (layer "B.Cu") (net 33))
 (segment (start 63.38 37.52) (end 63.38 80.52) (width 1) (layer "B.Cu") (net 33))
 (segment (start 115.38 40) (end 106.38 31) (width 1) (layer "B.Cu") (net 33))
 (segment (start 63.38 80.52) (end 65.38 82.52) (width 1) (layer "B.Cu") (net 33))
 (segment (start 74.38 77.52) (end 74.38 59.06) (width 1) (layer "B.Cu") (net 33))
 (segment (start 122.38 55.76) (end 115.38 48.76) (width 1) (layer "B.Cu") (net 33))
 (segment (start 69.38 82.52) (end 74.38 77.52) (width 1) (layer "B.Cu") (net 33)))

